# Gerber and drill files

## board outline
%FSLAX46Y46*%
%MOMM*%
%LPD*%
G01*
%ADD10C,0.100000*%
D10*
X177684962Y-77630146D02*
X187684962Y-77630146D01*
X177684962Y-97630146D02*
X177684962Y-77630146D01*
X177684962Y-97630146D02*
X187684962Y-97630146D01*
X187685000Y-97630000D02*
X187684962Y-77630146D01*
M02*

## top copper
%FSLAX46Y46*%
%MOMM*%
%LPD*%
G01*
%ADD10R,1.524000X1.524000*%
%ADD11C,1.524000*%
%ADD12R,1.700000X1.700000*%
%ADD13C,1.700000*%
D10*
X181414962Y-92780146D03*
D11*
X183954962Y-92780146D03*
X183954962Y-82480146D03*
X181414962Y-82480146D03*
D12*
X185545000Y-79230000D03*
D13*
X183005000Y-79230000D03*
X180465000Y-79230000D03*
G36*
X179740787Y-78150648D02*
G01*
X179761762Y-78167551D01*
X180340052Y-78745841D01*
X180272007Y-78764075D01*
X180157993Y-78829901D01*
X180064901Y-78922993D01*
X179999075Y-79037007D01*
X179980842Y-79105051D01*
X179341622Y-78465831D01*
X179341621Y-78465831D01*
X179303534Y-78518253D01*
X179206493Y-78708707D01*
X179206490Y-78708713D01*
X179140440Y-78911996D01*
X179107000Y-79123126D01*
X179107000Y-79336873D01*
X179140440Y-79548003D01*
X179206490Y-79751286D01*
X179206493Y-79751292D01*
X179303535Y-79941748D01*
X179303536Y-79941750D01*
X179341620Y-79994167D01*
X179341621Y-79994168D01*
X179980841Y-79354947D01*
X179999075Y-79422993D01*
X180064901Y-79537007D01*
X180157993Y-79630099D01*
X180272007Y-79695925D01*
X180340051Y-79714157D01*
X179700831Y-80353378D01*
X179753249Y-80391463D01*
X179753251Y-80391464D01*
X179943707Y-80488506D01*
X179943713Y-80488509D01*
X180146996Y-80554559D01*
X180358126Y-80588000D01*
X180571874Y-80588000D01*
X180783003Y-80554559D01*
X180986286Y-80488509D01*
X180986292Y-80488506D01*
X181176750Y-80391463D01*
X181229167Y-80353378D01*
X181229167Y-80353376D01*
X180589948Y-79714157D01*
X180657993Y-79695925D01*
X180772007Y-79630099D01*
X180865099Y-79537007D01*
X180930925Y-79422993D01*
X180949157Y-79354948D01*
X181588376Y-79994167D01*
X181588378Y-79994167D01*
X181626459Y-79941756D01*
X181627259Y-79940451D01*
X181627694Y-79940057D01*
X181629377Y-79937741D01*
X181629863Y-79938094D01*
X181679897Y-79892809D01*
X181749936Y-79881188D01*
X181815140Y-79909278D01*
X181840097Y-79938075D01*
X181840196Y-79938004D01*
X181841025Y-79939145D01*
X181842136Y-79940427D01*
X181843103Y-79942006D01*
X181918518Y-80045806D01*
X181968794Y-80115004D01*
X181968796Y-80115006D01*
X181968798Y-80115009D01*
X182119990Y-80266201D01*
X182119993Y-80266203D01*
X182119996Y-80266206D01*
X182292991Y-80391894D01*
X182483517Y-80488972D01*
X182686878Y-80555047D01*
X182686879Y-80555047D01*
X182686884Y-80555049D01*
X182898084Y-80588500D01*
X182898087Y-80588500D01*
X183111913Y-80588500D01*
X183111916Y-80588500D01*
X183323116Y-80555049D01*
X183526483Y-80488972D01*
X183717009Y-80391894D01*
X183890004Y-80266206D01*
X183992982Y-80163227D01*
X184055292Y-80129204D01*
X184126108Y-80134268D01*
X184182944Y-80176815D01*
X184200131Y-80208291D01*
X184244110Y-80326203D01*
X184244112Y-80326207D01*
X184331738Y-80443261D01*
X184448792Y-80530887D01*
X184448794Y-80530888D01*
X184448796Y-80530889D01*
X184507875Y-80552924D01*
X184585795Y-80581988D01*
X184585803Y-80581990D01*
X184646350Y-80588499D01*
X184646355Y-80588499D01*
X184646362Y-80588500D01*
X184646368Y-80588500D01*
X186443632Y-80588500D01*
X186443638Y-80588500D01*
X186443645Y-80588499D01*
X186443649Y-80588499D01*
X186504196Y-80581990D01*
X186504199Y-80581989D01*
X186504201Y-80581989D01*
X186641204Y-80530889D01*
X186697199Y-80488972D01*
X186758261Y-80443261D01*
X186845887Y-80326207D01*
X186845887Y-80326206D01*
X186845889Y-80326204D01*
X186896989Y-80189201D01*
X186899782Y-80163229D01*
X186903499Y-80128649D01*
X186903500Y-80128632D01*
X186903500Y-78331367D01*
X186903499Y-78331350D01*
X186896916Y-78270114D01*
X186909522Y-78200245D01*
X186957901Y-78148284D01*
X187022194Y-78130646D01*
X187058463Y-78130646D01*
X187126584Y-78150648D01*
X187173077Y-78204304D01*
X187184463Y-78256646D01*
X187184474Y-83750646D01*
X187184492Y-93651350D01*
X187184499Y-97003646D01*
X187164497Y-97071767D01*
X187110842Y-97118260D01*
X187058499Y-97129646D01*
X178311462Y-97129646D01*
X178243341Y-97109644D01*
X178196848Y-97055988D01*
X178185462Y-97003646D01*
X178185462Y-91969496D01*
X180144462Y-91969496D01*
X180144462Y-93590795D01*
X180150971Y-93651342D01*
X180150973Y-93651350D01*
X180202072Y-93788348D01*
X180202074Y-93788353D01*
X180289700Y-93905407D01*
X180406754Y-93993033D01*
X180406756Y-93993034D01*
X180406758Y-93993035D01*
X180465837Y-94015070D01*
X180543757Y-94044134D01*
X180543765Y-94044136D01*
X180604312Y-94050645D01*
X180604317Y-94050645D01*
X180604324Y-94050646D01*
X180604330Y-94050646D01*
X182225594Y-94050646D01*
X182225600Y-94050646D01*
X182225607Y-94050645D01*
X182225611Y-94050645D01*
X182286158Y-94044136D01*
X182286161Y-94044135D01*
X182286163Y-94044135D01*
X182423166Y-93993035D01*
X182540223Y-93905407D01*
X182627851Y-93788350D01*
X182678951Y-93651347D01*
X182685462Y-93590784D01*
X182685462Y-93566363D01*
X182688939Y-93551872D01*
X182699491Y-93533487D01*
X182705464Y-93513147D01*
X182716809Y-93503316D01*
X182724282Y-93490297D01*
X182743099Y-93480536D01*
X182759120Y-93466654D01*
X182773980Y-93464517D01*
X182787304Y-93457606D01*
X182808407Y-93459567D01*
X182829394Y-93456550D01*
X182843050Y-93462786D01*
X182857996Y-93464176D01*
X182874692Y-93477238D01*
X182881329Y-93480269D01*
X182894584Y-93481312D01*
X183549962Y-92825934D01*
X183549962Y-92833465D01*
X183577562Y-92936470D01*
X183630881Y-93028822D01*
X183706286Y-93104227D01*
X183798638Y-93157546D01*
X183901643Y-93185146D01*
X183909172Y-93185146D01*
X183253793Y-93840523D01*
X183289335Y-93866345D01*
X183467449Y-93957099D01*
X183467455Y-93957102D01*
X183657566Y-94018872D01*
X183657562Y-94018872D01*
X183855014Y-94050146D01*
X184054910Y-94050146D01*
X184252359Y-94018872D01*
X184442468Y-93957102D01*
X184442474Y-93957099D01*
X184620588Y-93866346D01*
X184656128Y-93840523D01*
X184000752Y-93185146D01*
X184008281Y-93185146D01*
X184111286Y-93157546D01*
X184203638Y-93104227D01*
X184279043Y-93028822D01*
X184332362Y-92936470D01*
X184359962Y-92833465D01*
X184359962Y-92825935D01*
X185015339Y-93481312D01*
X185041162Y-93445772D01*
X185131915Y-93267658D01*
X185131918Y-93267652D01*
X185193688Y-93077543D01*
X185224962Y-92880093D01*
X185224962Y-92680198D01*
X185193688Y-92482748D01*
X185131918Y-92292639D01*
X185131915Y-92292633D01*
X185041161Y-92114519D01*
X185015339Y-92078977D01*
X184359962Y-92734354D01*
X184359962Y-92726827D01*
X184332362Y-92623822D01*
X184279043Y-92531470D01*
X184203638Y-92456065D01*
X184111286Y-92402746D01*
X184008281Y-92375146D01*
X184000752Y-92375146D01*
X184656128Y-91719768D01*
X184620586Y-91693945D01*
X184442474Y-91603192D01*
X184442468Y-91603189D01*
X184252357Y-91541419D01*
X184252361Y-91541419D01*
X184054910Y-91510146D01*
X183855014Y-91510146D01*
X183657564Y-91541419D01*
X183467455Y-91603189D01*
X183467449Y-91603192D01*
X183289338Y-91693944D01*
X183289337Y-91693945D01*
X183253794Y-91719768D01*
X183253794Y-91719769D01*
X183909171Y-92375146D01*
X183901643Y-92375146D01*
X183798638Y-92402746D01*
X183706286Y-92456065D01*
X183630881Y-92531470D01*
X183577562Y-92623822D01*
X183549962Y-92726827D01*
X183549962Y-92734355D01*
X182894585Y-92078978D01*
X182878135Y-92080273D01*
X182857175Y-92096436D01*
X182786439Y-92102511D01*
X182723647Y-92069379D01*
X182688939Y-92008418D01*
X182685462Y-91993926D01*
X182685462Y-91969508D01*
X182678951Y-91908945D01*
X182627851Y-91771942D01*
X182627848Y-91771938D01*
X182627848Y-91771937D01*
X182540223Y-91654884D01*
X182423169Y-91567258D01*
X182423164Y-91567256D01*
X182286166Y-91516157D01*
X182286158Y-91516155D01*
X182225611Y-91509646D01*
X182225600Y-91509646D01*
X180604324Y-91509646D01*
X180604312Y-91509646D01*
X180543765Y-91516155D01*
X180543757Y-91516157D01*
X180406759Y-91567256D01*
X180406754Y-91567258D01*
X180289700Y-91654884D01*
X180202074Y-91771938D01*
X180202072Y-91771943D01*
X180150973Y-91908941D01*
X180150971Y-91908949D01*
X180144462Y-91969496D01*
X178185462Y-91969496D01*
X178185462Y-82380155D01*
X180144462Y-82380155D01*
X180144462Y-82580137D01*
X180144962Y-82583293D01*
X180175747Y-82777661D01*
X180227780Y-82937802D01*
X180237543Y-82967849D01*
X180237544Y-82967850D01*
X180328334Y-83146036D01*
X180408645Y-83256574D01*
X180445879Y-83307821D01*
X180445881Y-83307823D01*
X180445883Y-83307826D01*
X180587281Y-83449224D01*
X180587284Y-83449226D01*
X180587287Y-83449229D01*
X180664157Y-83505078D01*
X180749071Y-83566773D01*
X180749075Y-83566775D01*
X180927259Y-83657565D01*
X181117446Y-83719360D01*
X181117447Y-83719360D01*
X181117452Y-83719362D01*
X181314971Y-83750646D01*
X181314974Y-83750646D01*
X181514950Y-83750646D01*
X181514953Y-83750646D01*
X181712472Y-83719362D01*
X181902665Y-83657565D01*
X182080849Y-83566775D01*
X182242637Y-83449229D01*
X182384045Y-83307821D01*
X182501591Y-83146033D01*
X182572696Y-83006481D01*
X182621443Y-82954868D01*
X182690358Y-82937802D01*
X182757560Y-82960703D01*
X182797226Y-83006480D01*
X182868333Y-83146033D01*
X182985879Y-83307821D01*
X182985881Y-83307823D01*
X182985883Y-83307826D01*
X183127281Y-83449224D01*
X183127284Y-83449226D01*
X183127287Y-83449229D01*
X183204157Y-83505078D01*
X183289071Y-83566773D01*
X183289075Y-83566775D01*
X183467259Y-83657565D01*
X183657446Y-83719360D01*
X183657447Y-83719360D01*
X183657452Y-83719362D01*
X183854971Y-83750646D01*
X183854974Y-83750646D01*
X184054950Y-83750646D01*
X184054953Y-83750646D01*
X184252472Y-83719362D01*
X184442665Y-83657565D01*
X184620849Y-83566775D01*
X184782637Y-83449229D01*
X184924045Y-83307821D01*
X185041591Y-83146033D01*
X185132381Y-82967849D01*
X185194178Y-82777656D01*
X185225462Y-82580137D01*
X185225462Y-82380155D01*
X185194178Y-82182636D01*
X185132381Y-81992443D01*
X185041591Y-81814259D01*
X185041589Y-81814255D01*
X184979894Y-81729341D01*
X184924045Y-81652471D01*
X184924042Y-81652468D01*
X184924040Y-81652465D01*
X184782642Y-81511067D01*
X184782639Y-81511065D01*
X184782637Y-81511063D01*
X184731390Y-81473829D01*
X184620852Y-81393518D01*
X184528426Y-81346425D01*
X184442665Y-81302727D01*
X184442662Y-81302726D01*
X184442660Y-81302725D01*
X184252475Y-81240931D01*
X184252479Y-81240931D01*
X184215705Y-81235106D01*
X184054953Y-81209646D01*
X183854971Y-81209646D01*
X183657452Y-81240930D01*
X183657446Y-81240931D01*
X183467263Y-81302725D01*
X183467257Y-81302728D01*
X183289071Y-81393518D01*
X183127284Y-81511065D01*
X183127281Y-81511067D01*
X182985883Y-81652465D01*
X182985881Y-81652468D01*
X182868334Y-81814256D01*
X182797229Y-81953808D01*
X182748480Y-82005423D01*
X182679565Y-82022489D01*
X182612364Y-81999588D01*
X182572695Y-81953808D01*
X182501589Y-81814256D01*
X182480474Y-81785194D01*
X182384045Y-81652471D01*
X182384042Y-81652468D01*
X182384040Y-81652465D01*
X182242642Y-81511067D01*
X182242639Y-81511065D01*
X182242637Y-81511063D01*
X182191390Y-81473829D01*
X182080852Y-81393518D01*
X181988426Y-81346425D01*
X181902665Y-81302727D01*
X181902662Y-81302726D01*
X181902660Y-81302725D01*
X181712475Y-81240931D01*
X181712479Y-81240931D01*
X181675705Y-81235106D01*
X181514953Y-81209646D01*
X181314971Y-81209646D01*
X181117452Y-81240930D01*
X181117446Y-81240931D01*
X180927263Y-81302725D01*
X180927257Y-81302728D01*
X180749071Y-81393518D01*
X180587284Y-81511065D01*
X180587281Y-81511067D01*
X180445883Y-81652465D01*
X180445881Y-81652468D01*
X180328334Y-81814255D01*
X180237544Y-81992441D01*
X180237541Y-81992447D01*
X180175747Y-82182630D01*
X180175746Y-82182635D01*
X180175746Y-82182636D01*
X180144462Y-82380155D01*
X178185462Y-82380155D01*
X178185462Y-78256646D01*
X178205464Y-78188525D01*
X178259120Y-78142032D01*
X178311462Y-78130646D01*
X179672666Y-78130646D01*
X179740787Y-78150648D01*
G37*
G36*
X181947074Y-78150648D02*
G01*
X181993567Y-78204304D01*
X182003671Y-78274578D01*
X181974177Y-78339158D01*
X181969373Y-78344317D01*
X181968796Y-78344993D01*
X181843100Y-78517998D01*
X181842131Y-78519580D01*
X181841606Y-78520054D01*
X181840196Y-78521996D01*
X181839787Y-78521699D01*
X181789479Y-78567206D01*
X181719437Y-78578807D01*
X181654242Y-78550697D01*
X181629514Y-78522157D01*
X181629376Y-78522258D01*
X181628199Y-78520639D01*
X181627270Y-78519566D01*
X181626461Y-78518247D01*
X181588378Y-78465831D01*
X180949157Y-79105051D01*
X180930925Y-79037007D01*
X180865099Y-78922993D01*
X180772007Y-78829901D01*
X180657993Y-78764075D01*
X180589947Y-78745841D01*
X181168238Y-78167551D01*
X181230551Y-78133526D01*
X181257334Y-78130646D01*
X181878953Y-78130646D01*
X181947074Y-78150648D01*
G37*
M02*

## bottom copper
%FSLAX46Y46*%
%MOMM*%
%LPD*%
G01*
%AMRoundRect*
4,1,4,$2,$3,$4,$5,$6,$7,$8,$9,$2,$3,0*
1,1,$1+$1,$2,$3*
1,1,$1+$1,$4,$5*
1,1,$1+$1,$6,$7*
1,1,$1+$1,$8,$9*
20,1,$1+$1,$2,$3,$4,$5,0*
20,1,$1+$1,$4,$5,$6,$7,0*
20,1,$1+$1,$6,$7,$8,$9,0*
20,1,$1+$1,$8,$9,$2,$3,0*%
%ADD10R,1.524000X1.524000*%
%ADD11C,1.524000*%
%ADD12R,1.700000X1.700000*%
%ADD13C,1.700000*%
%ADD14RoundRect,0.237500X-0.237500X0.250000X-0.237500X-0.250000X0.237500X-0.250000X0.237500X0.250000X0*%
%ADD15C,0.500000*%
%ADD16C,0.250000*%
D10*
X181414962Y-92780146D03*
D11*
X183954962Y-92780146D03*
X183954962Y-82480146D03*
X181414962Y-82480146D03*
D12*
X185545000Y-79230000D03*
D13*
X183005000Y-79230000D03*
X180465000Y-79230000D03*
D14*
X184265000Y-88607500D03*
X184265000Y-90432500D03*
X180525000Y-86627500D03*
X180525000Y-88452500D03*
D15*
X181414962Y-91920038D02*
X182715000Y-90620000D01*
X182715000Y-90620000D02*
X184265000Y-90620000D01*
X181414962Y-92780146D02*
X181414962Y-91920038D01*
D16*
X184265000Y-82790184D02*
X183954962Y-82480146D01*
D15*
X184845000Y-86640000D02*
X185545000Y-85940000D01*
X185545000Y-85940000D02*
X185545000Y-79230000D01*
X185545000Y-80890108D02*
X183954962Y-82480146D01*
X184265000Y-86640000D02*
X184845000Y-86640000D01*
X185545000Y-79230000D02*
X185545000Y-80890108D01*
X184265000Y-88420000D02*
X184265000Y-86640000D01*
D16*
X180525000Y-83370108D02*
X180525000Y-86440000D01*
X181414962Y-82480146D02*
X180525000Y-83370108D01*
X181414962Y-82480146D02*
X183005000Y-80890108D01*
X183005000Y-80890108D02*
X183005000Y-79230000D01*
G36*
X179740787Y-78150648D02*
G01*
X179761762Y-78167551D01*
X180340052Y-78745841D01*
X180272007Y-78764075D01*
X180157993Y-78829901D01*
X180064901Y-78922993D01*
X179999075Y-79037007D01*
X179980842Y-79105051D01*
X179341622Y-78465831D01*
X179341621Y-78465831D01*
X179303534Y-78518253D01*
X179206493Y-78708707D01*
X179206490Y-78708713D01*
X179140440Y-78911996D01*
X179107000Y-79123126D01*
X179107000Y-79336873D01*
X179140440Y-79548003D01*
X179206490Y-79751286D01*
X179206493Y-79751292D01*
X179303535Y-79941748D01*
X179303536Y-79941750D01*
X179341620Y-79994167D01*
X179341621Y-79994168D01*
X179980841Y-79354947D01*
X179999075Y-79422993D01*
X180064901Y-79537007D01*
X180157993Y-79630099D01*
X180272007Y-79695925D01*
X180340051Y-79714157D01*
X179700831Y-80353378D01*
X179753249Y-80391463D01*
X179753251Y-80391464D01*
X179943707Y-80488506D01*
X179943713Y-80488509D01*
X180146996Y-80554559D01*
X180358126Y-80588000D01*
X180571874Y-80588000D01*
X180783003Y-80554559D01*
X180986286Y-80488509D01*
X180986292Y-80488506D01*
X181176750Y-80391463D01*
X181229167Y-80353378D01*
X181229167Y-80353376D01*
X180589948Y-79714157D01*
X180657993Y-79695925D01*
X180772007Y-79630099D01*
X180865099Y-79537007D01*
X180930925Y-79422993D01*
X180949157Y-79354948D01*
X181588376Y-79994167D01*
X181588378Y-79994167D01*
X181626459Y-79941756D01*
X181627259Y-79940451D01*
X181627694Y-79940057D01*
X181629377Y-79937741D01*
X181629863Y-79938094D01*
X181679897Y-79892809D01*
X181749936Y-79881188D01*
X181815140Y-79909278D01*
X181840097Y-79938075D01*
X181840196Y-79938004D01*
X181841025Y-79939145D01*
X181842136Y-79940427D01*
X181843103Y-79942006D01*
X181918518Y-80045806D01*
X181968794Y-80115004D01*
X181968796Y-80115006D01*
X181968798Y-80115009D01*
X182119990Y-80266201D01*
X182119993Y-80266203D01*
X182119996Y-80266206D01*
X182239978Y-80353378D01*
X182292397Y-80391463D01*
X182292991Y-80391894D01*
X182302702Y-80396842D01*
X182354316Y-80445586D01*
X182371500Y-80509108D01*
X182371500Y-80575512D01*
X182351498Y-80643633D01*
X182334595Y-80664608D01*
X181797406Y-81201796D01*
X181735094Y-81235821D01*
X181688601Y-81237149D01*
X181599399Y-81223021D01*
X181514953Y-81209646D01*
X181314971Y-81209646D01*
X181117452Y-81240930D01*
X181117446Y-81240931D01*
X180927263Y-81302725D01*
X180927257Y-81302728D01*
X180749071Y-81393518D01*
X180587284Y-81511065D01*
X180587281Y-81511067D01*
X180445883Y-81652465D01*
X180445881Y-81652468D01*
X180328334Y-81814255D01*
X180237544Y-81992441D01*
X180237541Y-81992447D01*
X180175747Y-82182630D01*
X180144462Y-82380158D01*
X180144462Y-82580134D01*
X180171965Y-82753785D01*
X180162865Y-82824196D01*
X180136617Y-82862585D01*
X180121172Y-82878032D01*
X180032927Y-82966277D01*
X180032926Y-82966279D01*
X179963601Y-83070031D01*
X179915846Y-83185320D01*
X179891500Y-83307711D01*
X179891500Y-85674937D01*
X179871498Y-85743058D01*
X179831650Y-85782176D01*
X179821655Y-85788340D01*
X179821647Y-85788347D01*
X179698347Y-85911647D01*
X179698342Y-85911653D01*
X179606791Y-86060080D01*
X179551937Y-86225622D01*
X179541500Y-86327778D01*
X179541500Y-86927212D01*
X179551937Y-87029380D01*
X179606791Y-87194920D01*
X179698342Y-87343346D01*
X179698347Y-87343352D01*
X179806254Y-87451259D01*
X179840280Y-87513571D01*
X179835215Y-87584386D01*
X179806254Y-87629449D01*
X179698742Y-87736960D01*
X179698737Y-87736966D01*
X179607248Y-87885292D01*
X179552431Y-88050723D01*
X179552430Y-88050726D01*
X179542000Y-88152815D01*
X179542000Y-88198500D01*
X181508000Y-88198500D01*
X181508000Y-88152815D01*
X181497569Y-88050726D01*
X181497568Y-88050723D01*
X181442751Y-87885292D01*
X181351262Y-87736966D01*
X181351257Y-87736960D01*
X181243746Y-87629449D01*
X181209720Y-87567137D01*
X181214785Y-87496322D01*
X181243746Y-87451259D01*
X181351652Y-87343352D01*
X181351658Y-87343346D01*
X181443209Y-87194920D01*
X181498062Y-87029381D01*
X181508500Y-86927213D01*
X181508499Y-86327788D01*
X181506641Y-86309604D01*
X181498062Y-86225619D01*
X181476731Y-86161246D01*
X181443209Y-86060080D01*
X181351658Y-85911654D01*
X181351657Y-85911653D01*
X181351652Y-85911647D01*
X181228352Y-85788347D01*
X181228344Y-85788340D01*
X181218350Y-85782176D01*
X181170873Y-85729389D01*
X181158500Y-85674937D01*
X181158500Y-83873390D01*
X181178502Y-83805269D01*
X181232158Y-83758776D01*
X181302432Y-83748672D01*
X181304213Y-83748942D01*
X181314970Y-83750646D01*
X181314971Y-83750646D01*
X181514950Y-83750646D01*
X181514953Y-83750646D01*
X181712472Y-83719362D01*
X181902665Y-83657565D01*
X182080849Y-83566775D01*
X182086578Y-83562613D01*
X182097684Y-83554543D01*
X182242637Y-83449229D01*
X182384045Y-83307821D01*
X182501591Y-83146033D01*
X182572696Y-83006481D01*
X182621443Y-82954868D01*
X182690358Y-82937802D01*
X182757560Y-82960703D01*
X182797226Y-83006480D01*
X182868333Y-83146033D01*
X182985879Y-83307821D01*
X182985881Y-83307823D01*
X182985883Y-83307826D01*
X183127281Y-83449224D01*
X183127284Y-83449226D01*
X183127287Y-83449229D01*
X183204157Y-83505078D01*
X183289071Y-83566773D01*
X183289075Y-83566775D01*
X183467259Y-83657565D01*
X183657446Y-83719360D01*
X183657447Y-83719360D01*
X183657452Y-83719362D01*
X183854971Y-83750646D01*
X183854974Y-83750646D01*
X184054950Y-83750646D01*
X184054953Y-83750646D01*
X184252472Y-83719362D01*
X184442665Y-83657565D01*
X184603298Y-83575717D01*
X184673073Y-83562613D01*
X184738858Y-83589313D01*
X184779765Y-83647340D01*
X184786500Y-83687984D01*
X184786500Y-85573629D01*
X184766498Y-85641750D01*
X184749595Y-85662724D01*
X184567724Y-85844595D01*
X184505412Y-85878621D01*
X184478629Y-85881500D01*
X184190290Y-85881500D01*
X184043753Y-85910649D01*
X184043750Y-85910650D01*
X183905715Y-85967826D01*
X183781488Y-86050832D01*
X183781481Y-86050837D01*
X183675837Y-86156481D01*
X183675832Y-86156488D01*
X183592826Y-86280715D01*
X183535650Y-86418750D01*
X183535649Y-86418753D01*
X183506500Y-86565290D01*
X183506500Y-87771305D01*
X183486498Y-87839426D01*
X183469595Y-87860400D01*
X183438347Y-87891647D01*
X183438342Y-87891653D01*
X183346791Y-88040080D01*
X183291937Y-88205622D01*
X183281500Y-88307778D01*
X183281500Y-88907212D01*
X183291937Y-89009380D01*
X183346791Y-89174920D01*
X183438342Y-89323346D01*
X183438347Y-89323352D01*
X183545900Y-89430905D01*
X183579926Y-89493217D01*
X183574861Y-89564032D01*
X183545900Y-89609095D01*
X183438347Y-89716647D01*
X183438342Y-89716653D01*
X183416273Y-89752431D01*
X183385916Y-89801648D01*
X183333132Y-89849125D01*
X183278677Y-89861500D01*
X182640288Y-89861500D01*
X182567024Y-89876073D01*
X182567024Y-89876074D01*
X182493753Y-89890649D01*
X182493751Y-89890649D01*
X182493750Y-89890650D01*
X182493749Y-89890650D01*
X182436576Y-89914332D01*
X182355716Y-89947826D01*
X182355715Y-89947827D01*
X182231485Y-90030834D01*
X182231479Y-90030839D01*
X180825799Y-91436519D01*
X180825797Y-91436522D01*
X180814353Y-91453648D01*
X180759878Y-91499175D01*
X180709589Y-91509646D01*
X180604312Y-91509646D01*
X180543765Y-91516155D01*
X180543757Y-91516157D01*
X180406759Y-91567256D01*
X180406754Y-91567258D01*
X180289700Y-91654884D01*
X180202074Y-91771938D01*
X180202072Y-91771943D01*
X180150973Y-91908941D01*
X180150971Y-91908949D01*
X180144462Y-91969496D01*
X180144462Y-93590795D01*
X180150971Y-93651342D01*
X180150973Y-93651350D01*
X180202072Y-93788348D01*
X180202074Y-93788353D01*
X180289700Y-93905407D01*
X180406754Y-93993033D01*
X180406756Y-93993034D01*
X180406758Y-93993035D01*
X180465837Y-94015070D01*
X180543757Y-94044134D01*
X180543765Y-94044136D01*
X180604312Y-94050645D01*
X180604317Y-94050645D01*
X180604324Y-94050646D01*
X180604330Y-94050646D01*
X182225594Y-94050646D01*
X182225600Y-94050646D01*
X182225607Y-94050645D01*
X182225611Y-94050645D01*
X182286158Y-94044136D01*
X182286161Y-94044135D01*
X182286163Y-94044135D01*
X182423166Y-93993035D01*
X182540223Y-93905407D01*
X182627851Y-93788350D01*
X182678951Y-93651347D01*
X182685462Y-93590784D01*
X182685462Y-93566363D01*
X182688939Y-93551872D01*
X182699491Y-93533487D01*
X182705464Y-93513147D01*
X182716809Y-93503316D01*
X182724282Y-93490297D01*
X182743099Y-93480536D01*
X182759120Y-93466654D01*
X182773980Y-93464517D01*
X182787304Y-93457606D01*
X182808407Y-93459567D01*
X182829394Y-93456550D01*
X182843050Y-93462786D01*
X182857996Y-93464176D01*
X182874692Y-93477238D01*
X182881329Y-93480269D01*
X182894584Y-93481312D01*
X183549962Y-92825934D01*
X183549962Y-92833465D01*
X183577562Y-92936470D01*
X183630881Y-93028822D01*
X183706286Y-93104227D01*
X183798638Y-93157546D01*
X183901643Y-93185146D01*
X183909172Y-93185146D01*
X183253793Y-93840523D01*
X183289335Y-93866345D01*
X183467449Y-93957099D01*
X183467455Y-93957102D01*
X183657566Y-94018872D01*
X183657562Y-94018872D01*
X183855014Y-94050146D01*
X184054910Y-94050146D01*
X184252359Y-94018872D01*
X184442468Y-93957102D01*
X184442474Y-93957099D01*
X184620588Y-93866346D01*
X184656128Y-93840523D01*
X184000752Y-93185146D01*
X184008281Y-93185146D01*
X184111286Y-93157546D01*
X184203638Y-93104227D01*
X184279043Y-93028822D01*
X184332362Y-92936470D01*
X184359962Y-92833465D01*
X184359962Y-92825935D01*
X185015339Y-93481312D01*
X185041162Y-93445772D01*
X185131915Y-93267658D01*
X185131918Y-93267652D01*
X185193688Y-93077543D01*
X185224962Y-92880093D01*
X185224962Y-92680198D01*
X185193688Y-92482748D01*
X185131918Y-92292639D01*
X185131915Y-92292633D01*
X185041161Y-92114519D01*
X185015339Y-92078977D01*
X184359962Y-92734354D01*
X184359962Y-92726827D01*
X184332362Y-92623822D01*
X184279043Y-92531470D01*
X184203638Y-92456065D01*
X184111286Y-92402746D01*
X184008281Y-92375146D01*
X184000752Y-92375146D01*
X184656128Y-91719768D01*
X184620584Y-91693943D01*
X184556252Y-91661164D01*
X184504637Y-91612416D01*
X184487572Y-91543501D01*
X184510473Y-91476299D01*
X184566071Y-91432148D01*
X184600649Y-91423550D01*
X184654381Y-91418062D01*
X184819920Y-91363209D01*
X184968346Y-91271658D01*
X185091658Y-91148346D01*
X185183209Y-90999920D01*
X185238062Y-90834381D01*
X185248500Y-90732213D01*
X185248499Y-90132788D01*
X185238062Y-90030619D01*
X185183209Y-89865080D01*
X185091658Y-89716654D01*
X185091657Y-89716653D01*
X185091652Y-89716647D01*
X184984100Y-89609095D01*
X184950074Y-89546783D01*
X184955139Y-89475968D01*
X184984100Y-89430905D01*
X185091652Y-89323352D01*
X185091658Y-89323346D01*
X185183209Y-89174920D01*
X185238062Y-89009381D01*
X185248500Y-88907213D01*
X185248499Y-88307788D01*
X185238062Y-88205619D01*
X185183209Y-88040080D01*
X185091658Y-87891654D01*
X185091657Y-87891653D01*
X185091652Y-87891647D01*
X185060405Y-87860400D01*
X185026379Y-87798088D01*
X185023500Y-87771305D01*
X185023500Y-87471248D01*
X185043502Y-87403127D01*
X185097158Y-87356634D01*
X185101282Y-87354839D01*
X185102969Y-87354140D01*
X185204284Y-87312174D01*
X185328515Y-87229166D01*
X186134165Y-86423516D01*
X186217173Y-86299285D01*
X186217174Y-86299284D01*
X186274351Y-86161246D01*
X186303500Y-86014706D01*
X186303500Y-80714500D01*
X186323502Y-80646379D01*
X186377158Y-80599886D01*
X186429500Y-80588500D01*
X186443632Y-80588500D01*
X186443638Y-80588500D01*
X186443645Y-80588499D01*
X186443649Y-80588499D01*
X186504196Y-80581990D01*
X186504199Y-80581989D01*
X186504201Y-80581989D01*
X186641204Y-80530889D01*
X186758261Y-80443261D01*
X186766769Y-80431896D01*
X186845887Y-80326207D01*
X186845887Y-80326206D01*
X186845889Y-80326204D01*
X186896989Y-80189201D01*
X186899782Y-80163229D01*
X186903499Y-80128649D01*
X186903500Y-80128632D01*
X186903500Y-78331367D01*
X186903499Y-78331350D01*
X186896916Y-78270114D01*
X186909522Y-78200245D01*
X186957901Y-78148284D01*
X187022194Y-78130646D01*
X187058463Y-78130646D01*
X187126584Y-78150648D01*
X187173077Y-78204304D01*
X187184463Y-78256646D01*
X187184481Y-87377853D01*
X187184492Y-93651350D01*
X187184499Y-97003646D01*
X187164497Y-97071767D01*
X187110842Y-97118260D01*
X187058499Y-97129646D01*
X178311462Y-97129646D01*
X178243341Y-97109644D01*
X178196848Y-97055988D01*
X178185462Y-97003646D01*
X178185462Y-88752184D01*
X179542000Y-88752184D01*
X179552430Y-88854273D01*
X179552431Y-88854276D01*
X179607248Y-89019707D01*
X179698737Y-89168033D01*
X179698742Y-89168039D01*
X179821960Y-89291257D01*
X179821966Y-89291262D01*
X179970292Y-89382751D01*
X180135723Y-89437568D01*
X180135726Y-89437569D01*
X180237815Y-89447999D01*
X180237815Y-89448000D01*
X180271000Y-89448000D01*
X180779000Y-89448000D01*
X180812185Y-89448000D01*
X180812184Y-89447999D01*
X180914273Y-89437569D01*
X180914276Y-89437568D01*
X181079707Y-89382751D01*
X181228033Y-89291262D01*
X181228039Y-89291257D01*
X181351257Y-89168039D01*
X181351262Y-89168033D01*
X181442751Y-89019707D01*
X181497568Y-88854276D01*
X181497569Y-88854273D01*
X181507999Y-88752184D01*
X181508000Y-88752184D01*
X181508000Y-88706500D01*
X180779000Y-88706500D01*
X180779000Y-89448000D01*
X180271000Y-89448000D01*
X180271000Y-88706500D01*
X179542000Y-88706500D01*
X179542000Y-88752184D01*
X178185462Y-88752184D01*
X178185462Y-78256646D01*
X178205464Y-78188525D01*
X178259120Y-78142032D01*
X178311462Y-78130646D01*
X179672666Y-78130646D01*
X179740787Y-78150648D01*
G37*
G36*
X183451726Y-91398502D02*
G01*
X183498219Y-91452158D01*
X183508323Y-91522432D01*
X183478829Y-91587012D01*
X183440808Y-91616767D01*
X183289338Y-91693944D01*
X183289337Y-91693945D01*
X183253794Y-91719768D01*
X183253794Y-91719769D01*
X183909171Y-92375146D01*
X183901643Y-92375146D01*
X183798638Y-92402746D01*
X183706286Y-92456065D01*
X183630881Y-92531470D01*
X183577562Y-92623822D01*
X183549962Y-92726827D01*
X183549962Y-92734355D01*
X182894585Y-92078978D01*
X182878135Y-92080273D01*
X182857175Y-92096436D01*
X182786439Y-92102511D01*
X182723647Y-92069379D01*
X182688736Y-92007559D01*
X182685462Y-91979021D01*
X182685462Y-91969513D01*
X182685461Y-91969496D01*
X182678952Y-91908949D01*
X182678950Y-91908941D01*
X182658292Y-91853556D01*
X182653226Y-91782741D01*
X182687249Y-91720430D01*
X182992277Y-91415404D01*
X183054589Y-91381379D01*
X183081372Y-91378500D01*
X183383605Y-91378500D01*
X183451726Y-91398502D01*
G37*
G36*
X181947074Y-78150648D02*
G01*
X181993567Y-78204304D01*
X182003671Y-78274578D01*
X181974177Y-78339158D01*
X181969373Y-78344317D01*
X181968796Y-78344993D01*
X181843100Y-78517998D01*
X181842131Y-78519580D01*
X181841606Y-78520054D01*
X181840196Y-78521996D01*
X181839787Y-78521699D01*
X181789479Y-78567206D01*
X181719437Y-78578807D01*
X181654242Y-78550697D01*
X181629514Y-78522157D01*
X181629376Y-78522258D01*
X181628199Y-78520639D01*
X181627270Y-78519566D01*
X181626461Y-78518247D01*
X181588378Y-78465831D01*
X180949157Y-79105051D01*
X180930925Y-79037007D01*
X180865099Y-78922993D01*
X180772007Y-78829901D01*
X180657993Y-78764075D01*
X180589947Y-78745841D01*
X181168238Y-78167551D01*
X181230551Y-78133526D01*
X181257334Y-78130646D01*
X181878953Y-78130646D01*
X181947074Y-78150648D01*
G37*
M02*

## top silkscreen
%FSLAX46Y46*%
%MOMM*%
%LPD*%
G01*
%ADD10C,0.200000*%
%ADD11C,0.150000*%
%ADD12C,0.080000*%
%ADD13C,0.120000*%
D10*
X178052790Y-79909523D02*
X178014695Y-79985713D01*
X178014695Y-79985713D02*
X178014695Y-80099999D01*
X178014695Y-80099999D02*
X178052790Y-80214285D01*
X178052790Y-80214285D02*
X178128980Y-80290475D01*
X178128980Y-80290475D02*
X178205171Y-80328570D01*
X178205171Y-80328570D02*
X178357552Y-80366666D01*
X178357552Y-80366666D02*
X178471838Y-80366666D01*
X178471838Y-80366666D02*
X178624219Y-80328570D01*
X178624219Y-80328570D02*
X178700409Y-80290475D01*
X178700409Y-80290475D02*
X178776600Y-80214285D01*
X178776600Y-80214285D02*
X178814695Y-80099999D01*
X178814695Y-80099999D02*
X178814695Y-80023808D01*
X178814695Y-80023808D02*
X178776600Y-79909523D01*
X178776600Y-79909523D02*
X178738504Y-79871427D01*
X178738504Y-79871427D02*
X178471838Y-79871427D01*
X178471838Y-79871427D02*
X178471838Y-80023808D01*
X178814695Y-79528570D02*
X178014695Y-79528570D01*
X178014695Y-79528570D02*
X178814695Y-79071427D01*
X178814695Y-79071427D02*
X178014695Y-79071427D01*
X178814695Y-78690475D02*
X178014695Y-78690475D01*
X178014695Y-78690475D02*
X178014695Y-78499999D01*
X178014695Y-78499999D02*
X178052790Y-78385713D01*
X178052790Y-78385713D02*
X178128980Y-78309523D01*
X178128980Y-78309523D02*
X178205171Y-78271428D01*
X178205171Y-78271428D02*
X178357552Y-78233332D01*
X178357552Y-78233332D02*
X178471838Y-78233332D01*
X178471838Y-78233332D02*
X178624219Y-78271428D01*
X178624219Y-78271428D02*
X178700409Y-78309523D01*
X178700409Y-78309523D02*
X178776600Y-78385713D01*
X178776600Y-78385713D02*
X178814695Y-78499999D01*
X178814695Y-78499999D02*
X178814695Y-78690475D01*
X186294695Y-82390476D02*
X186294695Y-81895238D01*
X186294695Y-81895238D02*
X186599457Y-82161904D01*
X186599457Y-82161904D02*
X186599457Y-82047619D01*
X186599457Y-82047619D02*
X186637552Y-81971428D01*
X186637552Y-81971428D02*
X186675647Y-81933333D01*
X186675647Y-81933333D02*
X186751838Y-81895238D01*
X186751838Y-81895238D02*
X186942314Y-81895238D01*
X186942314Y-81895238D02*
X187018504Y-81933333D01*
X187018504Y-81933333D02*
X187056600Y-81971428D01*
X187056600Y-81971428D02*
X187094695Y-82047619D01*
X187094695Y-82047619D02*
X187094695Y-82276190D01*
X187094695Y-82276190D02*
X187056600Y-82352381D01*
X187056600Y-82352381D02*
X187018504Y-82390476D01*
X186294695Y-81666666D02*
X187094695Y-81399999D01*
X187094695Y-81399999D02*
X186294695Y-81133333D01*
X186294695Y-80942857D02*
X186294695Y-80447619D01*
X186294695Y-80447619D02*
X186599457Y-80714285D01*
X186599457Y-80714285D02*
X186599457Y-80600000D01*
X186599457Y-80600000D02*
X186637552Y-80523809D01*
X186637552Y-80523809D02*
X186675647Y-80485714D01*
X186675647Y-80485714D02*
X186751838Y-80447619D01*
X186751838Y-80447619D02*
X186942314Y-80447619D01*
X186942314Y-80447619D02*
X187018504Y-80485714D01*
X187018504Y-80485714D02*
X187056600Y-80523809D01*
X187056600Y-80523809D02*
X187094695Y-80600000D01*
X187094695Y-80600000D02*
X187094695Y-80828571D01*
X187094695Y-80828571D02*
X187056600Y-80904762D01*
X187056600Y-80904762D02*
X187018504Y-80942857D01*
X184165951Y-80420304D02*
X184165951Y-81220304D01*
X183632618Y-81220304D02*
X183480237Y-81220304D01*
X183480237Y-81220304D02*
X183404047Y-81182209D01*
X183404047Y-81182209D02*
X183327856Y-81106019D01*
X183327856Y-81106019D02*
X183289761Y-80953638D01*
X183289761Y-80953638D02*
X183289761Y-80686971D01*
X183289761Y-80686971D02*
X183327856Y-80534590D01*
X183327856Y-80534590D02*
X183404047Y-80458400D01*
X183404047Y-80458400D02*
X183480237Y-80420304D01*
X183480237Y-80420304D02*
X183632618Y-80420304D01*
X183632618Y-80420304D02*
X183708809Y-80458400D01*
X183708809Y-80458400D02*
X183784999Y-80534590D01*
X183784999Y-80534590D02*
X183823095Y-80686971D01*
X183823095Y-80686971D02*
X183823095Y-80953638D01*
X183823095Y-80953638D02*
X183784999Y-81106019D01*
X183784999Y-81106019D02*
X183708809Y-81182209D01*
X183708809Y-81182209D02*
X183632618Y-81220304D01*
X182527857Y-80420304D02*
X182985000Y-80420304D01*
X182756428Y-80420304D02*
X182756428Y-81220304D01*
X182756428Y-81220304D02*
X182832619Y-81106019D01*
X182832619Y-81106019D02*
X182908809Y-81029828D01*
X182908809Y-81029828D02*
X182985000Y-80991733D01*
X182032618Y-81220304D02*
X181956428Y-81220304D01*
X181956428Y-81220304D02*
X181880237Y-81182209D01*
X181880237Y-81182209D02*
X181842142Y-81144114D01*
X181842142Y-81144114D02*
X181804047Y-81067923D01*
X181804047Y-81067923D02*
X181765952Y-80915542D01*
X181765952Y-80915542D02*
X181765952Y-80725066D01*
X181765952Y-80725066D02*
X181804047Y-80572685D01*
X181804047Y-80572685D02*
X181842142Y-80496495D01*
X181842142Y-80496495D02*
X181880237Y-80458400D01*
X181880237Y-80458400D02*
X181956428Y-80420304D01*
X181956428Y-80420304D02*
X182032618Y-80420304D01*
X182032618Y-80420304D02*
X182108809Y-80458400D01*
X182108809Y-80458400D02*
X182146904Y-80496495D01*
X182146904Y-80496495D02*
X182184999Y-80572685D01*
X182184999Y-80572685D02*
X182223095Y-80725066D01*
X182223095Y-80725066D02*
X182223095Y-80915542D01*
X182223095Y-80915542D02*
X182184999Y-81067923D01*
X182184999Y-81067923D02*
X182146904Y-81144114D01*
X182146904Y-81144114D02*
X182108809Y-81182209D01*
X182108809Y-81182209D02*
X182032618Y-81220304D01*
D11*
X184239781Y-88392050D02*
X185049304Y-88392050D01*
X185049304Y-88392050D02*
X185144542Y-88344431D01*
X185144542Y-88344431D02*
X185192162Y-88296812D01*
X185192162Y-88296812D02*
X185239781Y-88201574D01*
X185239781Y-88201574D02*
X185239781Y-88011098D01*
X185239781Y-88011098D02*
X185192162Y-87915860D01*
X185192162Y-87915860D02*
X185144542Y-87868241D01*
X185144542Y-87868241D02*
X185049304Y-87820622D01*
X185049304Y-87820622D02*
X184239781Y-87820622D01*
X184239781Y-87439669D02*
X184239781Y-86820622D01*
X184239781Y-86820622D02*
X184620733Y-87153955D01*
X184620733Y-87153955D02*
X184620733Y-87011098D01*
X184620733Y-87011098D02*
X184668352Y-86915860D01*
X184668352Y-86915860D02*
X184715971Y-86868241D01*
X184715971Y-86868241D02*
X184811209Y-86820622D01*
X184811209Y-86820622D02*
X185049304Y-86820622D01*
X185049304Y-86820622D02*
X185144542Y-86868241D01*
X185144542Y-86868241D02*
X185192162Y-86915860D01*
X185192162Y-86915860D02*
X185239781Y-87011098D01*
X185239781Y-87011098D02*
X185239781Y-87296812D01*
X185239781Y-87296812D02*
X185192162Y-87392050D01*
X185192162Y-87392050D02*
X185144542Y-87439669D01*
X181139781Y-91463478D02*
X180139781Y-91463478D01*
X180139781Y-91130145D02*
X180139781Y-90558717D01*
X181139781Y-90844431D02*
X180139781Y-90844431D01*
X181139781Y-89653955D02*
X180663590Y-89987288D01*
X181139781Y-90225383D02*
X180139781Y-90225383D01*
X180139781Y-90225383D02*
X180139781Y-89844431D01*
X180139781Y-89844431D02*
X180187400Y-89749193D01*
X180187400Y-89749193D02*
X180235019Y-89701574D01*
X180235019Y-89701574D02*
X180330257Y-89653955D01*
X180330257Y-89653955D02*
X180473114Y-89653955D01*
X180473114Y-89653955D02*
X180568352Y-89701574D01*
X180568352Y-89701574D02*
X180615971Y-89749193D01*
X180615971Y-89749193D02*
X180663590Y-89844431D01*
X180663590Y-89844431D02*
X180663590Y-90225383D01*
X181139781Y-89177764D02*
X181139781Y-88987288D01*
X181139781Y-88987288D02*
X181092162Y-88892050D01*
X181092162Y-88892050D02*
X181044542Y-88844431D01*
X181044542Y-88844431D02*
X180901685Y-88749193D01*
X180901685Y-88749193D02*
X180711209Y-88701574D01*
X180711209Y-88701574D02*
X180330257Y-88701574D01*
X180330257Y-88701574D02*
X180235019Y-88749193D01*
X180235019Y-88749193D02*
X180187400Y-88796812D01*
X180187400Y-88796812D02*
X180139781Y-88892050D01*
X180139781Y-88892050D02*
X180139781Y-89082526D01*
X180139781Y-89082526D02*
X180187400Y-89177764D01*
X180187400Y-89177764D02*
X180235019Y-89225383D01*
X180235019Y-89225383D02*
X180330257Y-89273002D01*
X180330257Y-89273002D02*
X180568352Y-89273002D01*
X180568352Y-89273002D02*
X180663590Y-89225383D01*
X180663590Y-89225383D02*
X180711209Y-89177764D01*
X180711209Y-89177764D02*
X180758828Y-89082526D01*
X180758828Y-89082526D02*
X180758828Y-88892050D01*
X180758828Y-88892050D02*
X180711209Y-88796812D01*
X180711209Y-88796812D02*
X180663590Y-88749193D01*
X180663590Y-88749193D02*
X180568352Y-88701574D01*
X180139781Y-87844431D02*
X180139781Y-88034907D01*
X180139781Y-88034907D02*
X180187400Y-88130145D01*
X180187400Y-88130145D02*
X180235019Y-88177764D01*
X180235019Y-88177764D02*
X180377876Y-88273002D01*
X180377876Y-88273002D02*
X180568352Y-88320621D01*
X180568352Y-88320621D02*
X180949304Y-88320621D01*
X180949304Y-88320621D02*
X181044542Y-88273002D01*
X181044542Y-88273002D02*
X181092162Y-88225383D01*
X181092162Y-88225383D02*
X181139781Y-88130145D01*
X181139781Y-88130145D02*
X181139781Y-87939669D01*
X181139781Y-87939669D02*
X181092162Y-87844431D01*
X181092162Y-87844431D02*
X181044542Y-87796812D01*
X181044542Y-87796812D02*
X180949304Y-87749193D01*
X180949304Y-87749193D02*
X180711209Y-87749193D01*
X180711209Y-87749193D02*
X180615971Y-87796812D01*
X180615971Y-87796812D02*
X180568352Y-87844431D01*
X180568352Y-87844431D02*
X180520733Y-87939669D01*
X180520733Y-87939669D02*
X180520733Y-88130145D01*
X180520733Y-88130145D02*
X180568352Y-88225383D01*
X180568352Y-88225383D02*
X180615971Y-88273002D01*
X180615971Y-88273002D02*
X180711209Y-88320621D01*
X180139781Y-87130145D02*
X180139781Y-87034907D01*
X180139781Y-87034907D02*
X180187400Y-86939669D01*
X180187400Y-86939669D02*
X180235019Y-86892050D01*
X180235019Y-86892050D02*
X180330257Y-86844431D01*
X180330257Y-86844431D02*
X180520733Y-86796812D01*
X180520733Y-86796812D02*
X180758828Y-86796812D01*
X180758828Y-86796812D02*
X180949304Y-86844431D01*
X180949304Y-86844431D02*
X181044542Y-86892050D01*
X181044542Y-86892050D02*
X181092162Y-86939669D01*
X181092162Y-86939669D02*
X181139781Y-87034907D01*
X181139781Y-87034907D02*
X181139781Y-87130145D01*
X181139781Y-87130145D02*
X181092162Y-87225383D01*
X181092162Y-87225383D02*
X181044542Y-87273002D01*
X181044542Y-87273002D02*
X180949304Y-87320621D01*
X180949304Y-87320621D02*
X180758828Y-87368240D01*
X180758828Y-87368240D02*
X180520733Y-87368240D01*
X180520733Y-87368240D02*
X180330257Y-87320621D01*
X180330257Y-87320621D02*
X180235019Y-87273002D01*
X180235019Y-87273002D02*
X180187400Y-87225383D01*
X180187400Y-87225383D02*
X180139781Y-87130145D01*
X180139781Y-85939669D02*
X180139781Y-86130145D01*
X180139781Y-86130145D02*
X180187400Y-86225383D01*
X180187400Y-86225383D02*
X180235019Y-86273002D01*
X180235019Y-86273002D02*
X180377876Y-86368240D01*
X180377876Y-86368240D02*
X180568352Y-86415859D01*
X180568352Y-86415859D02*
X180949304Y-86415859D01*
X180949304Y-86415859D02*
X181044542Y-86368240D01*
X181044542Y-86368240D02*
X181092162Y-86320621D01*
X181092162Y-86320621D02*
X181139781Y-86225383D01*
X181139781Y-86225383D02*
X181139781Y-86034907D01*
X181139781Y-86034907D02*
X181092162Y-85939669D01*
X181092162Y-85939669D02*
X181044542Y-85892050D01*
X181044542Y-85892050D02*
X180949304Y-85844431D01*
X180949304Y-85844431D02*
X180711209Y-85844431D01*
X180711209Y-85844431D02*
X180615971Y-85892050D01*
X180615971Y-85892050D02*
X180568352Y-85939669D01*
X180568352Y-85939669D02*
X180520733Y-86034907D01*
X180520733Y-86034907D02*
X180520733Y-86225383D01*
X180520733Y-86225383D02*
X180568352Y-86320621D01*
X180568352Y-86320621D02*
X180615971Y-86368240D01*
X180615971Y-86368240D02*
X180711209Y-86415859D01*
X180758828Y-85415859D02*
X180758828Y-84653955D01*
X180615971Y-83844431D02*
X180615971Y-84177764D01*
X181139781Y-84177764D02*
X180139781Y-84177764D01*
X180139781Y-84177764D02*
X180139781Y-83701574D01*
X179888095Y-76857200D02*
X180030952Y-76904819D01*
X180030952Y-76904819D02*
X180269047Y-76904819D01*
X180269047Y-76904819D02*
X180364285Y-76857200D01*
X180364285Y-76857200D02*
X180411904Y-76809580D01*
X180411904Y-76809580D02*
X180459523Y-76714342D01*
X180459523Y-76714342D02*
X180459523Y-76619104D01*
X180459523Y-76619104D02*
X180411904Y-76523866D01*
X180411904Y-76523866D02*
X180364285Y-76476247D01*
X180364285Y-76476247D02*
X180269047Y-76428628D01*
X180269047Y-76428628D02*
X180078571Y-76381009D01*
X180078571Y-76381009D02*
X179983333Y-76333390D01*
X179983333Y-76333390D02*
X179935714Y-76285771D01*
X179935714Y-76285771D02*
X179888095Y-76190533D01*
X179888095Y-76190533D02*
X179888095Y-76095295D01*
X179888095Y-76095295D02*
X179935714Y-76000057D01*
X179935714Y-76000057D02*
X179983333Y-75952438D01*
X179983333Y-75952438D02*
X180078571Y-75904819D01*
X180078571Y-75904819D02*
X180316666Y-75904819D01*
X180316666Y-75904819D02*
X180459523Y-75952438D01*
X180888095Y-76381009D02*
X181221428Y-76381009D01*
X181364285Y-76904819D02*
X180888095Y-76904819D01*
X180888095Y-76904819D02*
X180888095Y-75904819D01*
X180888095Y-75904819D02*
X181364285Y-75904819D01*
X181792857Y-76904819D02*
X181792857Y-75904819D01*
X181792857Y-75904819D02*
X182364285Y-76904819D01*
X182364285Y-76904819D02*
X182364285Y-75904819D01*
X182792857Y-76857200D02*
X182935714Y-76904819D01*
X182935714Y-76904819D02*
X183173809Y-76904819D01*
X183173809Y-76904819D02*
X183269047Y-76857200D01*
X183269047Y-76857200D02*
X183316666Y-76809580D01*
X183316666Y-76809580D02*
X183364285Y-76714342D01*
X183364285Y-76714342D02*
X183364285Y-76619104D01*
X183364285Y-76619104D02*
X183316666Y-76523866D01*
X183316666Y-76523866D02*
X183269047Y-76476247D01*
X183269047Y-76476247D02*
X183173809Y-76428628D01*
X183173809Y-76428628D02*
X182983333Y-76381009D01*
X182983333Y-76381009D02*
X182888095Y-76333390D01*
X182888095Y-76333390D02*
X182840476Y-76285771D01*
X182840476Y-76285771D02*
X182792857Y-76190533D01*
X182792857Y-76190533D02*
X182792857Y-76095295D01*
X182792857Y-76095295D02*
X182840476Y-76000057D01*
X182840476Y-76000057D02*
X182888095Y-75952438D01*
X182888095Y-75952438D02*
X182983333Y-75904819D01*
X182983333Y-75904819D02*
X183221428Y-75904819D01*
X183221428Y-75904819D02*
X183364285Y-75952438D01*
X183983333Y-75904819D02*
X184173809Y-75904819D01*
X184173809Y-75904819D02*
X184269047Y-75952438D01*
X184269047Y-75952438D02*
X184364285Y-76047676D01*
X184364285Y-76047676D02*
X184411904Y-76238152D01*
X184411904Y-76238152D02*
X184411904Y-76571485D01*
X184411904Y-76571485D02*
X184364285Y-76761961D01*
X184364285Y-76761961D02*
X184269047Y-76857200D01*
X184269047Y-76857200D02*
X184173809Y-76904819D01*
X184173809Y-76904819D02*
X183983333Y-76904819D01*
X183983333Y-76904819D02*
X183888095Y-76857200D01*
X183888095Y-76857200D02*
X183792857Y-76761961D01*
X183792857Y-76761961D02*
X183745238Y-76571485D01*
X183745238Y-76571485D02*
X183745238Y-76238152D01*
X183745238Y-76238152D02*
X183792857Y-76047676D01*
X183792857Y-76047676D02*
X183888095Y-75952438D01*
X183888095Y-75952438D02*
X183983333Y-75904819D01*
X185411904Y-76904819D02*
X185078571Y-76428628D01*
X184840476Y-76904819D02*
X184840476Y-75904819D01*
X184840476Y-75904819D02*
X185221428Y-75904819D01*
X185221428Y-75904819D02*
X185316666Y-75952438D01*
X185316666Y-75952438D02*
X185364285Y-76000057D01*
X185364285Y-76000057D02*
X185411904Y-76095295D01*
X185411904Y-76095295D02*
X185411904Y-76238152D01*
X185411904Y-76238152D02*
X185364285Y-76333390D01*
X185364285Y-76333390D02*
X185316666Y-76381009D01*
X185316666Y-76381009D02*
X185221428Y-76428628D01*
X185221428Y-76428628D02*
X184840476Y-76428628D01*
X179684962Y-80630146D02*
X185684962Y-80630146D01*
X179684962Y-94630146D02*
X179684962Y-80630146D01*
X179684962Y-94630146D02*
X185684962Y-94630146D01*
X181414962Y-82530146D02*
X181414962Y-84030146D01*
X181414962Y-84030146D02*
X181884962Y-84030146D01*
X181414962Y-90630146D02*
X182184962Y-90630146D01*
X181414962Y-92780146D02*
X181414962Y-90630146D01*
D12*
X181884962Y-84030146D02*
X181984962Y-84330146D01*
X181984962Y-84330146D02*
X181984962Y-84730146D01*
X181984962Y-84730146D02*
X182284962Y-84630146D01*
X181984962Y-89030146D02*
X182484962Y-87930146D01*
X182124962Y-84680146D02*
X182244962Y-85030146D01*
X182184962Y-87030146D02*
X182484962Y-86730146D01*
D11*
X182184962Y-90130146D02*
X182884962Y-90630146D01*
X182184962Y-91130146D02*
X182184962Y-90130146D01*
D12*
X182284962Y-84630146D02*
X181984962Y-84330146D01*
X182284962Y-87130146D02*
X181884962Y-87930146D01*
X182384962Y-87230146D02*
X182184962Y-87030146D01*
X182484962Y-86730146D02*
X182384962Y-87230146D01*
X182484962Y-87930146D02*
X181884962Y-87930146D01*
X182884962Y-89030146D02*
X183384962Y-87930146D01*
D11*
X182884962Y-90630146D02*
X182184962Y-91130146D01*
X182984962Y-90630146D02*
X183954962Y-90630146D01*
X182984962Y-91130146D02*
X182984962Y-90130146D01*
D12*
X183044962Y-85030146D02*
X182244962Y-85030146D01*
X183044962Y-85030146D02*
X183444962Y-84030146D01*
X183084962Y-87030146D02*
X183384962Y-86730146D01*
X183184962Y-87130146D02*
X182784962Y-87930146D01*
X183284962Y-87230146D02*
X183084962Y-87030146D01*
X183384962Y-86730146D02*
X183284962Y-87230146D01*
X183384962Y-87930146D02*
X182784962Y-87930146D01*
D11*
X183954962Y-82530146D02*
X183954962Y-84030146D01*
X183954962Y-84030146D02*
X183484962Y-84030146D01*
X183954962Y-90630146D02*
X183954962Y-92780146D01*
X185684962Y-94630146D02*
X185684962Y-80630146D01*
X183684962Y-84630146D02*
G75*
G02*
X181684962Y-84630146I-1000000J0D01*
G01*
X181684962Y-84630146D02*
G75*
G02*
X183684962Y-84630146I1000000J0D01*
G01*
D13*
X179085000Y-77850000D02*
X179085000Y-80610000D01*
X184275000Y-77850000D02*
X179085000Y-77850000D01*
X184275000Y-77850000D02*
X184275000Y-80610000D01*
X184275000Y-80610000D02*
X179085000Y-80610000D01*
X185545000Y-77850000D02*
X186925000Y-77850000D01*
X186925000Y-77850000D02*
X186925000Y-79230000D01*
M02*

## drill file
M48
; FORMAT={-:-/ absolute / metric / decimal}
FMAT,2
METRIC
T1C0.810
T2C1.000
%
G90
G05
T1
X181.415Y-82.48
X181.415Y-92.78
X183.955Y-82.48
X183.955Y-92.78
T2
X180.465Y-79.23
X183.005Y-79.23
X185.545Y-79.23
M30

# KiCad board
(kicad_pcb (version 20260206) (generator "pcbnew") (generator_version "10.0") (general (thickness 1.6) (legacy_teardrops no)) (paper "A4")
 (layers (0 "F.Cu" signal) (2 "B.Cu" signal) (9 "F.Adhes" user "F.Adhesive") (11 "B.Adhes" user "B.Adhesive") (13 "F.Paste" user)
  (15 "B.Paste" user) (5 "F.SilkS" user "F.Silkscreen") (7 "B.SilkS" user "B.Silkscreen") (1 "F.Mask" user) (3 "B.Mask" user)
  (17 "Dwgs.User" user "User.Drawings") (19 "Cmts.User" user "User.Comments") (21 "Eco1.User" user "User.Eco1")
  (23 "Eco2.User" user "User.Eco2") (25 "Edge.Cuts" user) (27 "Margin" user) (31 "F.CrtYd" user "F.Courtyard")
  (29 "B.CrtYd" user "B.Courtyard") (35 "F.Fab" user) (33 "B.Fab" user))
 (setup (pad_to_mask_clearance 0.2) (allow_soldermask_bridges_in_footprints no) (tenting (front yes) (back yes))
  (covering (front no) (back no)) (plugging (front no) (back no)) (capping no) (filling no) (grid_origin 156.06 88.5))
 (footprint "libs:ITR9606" (layer "F.Cu") (at 182.684962 87.630146 90)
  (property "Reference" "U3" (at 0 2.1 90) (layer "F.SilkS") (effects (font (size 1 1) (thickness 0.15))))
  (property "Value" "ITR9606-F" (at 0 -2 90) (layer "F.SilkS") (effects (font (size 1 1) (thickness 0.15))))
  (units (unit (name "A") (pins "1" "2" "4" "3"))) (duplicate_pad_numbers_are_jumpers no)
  (fp_line (start 7 -3) (end 7 3) (stroke (width 0.15) (type solid)) (layer "F.SilkS"))
  (fp_line (start -7 -3) (end 7 -3) (stroke (width 0.15) (type solid)) (layer "F.SilkS"))
  (fp_line (start -7 -3) (end -7 3) (stroke (width 0.15) (type solid)) (layer "F.SilkS"))
  (fp_line (start 5.1 -1.27) (end 3.6 -1.27) (stroke (width 0.15) (type solid)) (layer "F.SilkS"))
  (fp_line (start 3.6 -1.27) (end 3.6 -0.8) (stroke (width 0.15) (type solid)) (layer "F.SilkS"))
  (fp_line (start -3 -1.27) (end -3 -0.5) (stroke (width 0.15) (type solid)) (layer "F.SilkS"))
  (fp_line (start -5.15 -1.27) (end -3 -1.27) (stroke (width 0.15) (type solid)) (layer "F.SilkS"))
  (fp_line (start 3.6 -0.8) (end 3.3 -0.7) (stroke (width 0.08) (type solid)) (layer "F.SilkS"))
  (fp_line (start 3.3 -0.7) (end 2.9 -0.7) (stroke (width 0.08) (type solid)) (layer "F.SilkS"))
  (fp_line (start 2.9 -0.7) (end 3 -0.4) (stroke (width 0.08) (type solid)) (layer "F.SilkS"))
  (fp_line (start -1.4 -0.7) (end -0.3 -0.2) (stroke (width 0.08) (type solid)) (layer "F.SilkS"))
  (fp_line (start 2.95 -0.56) (end 2.6 -0.44) (stroke (width 0.08) (type solid)) (layer "F.SilkS"))
  (fp_line (start 0.6 -0.5) (end 0.9 -0.2) (stroke (width 0.08) (type solid)) (layer "F.SilkS"))
  (fp_line (start -2.5 -0.5) (end -3 0.2) (stroke (width 0.15) (type solid)) (layer "F.SilkS"))
  (fp_line (start -3.5 -0.5) (end -2.5 -0.5) (stroke (width 0.15) (type solid)) (layer "F.SilkS"))
  (fp_line (start 3 -0.4) (end 3.3 -0.7) (stroke (width 0.08) (type solid)) (layer "F.SilkS"))
  (fp_line (start 0.5 -0.4) (end -0.3 -0.8) (stroke (width 0.08) (type solid)) (layer "F.SilkS"))
  (fp_line (start 0.4 -0.3) (end 0.6 -0.5) (stroke (width 0.08) (type solid)) (layer "F.SilkS"))
  (fp_line (start 0.9 -0.2) (end 0.4 -0.3) (stroke (width 0.08) (type solid)) (layer "F.SilkS"))
  (fp_line (start -0.3 -0.2) (end -0.3 -0.8) (stroke (width 0.08) (type solid)) (layer "F.SilkS"))
  (fp_line (start -1.4 0.2) (end -0.3 0.7) (stroke (width 0.08) (type solid)) (layer "F.SilkS"))
  (fp_line (start -3 0.2) (end -3.5 -0.5) (stroke (width 0.15) (type solid)) (layer "F.SilkS"))
  (fp_line (start -3 0.3) (end -3 1.27) (stroke (width 0.15) (type solid)) (layer "F.SilkS"))
  (fp_line (start -3.5 0.3) (end -2.5 0.3) (stroke (width 0.15) (type solid)) (layer "F.SilkS"))
  (fp_line (start 2.6 0.36) (end 2.6 -0.44) (stroke (width 0.08) (type solid)) (layer "F.SilkS"))
  (fp_line (start 2.6 0.36) (end 3.6 0.76) (stroke (width 0.08) (type solid)) (layer "F.SilkS"))
  (fp_line (start 0.6 0.4) (end 0.9 0.7) (stroke (width 0.08) (type solid)) (layer "F.SilkS"))
  (fp_line (start 0.5 0.5) (end -0.3 0.1) (stroke (width 0.08) (type solid)) (layer "F.SilkS"))
  (fp_line (start 0.4 0.6) (end 0.6 0.4) (stroke (width 0.08) (type solid)) (layer "F.SilkS"))
  (fp_line (start 0.9 0.7) (end 0.4 0.6) (stroke (width 0.08) (type solid)) (layer "F.SilkS"))
  (fp_line (start -0.3 0.7) (end -0.3 0.1) (stroke (width 0.08) (type solid)) (layer "F.SilkS"))
  (fp_line (start 5.1 1.27) (end 3.6 1.27) (stroke (width 0.15) (type solid)) (layer "F.SilkS"))
  (fp_line (start 3.6 1.27) (end 3.6 0.8) (stroke (width 0.15) (type solid)) (layer "F.SilkS"))
  (fp_line (start -3 1.27) (end -5.15 1.27) (stroke (width 0.15) (type solid)) (layer "F.SilkS"))
  (fp_line (start -7 3) (end 7 3) (stroke (width 0.15) (type solid)) (layer "F.SilkS"))
  (fp_circle (center 3 0) (end 4 0) (stroke (width 0.15) (type solid)) (fill no) (layer "F.SilkS"))
  (pad "1" thru_hole rect (at -5.15 -1.27 90) (size 1.524 1.524) (drill 0.81) (layers "*.Cu" "*.Mask") (remove_unused_layers no)
   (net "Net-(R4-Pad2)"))
  (pad "2" thru_hole circle (at -5.15 1.27 90) (size 1.524 1.524) (drill 0.81) (layers "*.Cu" "*.Mask") (remove_unused_layers no)
   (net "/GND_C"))
  (pad "3" thru_hole circle (at 5.15 1.27 90) (size 1.524 1.524) (drill 0.81) (layers "*.Cu" "*.Mask") (remove_unused_layers no)
   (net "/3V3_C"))
  (pad "4" thru_hole circle (at 5.15 -1.27 90) (size 1.524 1.524) (drill 0.81) (layers "*.Cu" "*.Mask") (remove_unused_layers no)
   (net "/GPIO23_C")))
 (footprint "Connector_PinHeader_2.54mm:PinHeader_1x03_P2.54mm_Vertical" (layer "F.Cu") (at 185.545 79.23 -90)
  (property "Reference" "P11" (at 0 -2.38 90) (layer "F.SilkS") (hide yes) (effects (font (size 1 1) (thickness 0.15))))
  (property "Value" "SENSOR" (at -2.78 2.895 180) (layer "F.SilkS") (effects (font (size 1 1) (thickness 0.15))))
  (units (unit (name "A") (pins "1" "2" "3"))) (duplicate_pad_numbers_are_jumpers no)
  (fp_line (start -1.38 6.46) (end 1.38 6.46) (stroke (width 0.12) (type solid)) (layer "F.SilkS"))
  (fp_line (start -1.38 1.27) (end -1.38 6.46) (stroke (width 0.12) (type solid)) (layer "F.SilkS"))
  (fp_line (start -1.38 1.27) (end 1.38 1.27) (stroke (width 0.12) (type solid)) (layer "F.SilkS"))
  (fp_line (start 1.38 1.27) (end 1.38 6.46) (stroke (width 0.12) (type solid)) (layer "F.SilkS"))
  (fp_line (start -1.38 0) (end -1.38 -1.38) (stroke (width 0.12) (type solid)) (layer "F.SilkS"))
  (fp_line (start -1.38 -1.38) (end 0 -1.38) (stroke (width 0.12) (type solid)) (layer "F.SilkS"))
  (pad "1" thru_hole rect (at 0 0 270) (size 1.7 1.7) (drill 1) (layers "*.Cu" "*.Mask") (remove_unused_layers no) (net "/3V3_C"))
  (pad "2" thru_hole circle (at 0 2.54 270) (size 1.7 1.7) (drill 1) (layers "*.Cu" "*.Mask") (remove_unused_layers no) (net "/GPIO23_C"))
  (pad "3" thru_hole circle (at 0 5.08 270) (size 1.7 1.7) (drill 1) (layers "*.Cu" "*.Mask") (remove_unused_layers no) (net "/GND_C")))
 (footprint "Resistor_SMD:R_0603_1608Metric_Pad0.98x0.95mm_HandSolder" (layer "B.Cu") (at 184.265 89.52 -90)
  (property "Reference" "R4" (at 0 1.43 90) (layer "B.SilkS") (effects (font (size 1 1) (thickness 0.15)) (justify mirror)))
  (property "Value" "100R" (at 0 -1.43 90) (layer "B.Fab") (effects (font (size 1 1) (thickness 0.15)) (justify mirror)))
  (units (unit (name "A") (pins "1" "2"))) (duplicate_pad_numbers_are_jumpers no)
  (pad "1" smd roundrect (at -0.9125 0 270) (size 0.975 0.95) (layers "B.Cu" "B.Mask" "B.Paste") (roundrect_rratio 0.25) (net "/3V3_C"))
  (pad "2" smd roundrect (at 0.9125 0 270) (size 0.975 0.95) (layers "B.Cu" "B.Mask" "B.Paste") (roundrect_rratio 0.25)
   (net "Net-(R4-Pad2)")))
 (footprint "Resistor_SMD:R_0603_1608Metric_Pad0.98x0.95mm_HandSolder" (layer "B.Cu") (at 180.525 87.54 -90)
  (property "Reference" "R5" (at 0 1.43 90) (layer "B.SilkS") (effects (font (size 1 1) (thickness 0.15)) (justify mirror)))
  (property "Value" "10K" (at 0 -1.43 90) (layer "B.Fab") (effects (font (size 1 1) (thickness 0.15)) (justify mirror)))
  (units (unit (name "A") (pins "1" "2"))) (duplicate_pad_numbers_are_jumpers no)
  (pad "1" smd roundrect (at -0.9125 0 270) (size 0.975 0.95) (layers "B.Cu" "B.Mask" "B.Paste") (roundrect_rratio 0.25) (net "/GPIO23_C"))
  (pad "2" smd roundrect (at 0.9125 0 270) (size 0.975 0.95) (layers "B.Cu" "B.Mask" "B.Paste") (roundrect_rratio 0.25) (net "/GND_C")))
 (gr_line (start 177.684962 77.630146) (end 187.684962 77.630146) (stroke (width 0.1) (type solid)) (layer "Edge.Cuts"))
 (gr_line (start 177.684962 97.630146) (end 177.684962 77.630146) (stroke (width 0.1) (type solid)) (layer "Edge.Cuts"))
 (gr_line (start 177.684962 97.630146) (end 187.684962 97.630146) (stroke (width 0.1) (type solid)) (layer "Edge.Cuts"))
 (gr_line (start 187.685 97.63) (end 187.684962 77.630146) (stroke (width 0.1) (type solid)) (layer "Edge.Cuts"))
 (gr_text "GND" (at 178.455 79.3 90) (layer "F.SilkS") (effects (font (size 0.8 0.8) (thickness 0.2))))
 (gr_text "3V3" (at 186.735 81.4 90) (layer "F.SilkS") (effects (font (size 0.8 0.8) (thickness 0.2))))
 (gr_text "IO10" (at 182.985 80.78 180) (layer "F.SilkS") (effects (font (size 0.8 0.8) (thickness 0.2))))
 (segment (start 181.414962 91.920038) (end 182.715 90.62) (width 0.5) (layer "B.Cu") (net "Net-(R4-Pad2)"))
 (segment (start 182.715 90.62) (end 184.265 90.62) (width 0.5) (layer "B.Cu") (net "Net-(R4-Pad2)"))
 (segment (start 181.414962 92.780146) (end 181.414962 91.920038) (width 0.5) (layer "B.Cu") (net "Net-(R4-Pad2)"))
 (segment (start 184.265 82.790184) (end 183.954962 82.480146) (width 0.25) (layer "B.Cu") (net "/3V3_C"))
 (segment (start 184.845 86.64) (end 185.545 85.94) (width 0.5) (layer "B.Cu") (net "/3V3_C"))
 (segment (start 185.545 85.94) (end 185.545 79.23) (width 0.5) (layer "B.Cu") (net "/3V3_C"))
 (segment (start 185.545 80.890108) (end 183.954962 82.480146) (width 0.5) (layer "B.Cu") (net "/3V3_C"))
 (segment (start 184.265 86.64) (end 184.845 86.64) (width 0.5) (layer "B.Cu") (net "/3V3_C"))
 (segment (start 185.545 79.23) (end 185.545 80.890108) (width 0.5) (layer "B.Cu") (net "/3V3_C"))
 (segment (start 184.265 88.42) (end 184.265 86.64) (width 0.5) (layer "B.Cu") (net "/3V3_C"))
 (segment (start 180.525 83.370108) (end 180.525 86.44) (width 0.25) (layer "B.Cu") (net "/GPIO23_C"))
 (segment (start 181.414962 82.480146) (end 180.525 83.370108) (width 0.25) (layer "B.Cu") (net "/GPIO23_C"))
 (segment (start 181.414962 82.480146) (end 183.005 80.890108) (width 0.25) (layer "B.Cu") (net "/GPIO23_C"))
 (segment (start 183.005 80.890108) (end 183.005 79.23) (width 0.25) (layer "B.Cu") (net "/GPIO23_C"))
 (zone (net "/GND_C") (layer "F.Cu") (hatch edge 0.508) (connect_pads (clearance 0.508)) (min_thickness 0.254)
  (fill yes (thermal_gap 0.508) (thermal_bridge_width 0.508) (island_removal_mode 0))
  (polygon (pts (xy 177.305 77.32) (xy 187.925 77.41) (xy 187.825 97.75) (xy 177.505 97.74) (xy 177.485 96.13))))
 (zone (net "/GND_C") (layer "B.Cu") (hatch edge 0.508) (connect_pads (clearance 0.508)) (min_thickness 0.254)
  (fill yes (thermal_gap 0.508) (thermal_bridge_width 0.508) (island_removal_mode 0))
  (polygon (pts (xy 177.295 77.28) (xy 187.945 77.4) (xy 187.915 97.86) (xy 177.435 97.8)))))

